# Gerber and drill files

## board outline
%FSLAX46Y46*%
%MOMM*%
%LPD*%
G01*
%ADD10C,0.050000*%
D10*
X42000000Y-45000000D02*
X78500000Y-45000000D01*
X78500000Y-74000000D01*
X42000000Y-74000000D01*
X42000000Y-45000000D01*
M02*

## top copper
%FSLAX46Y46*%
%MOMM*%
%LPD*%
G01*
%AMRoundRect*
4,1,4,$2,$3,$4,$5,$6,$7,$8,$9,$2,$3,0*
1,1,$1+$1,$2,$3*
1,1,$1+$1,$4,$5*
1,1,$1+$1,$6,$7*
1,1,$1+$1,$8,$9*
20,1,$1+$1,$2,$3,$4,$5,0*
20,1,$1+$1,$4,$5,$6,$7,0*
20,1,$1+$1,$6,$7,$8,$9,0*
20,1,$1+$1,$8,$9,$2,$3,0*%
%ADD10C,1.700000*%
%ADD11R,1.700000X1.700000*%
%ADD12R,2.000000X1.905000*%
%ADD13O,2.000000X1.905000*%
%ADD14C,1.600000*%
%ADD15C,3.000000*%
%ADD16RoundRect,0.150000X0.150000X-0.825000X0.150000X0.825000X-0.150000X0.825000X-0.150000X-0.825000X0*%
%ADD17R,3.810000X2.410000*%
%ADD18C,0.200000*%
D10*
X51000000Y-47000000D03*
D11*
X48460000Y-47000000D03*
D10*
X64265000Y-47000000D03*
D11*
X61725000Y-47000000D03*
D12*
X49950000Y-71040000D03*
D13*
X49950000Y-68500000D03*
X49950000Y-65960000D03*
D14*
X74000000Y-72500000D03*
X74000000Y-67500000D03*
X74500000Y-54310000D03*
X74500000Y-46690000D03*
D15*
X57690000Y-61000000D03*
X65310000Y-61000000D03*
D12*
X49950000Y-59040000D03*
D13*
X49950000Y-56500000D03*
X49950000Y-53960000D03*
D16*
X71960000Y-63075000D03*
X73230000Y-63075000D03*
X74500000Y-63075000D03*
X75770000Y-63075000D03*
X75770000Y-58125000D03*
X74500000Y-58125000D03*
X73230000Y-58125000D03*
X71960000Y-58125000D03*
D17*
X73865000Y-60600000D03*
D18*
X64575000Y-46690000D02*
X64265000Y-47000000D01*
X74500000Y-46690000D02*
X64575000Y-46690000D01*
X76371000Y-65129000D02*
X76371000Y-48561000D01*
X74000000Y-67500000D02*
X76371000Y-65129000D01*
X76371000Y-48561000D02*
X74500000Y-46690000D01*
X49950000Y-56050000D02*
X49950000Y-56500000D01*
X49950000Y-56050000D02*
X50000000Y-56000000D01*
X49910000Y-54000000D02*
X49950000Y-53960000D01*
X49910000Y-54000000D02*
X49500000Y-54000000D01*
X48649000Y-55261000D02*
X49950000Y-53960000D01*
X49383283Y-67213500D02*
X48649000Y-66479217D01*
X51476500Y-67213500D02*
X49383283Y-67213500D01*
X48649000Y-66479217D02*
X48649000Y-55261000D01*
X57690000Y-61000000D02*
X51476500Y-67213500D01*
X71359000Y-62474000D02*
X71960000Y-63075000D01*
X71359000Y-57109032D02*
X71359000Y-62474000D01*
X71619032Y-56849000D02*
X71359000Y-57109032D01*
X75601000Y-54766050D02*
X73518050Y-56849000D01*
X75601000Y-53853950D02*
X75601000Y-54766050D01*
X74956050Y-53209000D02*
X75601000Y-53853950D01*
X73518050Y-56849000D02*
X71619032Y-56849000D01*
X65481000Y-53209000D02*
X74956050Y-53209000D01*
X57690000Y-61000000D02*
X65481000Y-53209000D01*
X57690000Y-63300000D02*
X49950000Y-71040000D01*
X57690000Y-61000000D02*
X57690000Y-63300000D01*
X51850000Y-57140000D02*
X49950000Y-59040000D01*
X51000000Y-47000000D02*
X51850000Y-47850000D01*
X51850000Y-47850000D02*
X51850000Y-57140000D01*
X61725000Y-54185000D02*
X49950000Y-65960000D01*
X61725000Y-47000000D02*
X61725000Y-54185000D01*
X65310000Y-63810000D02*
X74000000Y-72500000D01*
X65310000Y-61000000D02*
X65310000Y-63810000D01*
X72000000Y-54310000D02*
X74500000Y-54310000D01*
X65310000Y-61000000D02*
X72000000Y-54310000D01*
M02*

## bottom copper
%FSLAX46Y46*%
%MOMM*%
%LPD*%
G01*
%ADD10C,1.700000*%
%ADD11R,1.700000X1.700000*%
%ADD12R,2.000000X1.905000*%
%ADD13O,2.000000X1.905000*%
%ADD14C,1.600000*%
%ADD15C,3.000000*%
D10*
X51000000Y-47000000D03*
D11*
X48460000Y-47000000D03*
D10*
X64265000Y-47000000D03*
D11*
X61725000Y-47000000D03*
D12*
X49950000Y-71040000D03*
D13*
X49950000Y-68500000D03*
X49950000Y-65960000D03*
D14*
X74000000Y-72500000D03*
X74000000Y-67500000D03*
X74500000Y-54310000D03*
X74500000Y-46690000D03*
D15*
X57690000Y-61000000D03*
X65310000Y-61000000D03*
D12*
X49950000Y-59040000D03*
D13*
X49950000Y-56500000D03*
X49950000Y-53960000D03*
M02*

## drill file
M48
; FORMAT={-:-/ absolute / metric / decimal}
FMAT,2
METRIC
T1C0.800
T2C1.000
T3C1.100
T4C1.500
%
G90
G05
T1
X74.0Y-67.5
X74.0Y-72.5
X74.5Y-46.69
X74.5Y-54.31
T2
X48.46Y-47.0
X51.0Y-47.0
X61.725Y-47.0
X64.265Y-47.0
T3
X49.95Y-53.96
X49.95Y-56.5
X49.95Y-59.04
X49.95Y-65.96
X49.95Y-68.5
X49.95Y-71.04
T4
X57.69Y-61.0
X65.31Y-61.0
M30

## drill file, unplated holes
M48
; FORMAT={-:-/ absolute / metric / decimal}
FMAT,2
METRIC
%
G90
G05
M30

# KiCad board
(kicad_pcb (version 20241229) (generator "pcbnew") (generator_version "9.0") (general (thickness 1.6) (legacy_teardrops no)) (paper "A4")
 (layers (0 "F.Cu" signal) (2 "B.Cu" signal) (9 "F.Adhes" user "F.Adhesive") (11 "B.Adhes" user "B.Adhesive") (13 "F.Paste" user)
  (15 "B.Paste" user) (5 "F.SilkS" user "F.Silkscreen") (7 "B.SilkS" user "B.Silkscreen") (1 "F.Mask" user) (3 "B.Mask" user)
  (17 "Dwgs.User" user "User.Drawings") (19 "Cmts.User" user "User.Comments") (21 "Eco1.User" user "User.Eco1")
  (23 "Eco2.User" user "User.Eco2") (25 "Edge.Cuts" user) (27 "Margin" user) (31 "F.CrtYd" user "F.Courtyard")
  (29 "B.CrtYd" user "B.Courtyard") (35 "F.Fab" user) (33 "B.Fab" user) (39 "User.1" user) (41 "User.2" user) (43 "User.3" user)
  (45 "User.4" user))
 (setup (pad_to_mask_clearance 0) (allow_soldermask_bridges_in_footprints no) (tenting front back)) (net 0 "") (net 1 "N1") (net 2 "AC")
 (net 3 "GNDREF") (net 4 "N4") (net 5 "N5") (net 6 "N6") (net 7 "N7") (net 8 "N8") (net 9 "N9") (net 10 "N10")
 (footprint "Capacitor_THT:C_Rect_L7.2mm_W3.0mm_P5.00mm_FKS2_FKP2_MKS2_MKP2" (layer "F.Cu") (at 74 72.5 90)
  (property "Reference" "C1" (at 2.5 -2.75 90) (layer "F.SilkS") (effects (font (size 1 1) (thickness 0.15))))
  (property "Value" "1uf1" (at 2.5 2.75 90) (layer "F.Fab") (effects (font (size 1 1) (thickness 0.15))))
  (pad "1" thru_hole circle (at 0 0 90) (size 1.6 1.6) (drill 0.8) (layers "*.Cu" "*.Mask") (remove_unused_layers no) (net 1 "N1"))
  (pad "2" thru_hole circle (at 5 0 90) (size 1.6 1.6) (drill 0.8) (layers "*.Cu" "*.Mask") (remove_unused_layers no) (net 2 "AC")))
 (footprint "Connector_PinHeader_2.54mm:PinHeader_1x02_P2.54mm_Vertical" (layer "F.Cu") (at 48.46 47 90)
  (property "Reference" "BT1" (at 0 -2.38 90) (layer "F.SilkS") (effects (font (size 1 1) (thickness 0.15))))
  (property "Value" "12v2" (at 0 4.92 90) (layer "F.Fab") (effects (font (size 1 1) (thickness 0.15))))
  (pad "1" thru_hole rect (at 0 0 90) (size 1.7 1.7) (drill 1) (layers "*.Cu" "*.Mask") (remove_unused_layers no) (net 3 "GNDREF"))
  (pad "2" thru_hole circle (at 0 2.54 90) (size 1.7 1.7) (drill 1) (layers "*.Cu" "*.Mask") (remove_unused_layers no) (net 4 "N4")))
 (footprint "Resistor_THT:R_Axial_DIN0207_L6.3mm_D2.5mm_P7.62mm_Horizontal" (layer "F.Cu") (at 74.5 54.31 90)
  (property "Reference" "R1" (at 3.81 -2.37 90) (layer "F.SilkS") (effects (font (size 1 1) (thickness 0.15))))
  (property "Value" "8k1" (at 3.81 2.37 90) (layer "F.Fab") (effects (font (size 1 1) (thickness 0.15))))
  (pad "1" thru_hole circle (at 0 0 90) (size 1.6 1.6) (drill 0.8) (layers "*.Cu" "*.Mask") (remove_unused_layers no) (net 1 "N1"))
  (pad "2" thru_hole circle (at 7.62 0 90) (size 1.6 1.6) (drill 0.8) (layers "*.Cu" "*.Mask") (remove_unused_layers no) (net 2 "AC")))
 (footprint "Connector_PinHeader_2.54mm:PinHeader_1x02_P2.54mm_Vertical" (layer "F.Cu") (at 61.725 47 90)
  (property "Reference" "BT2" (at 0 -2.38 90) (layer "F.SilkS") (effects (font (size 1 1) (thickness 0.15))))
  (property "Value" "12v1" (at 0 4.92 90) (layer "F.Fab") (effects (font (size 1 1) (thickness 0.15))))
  (pad "1" thru_hole rect (at 0 0 90) (size 1.7 1.7) (drill 1) (layers "*.Cu" "*.Mask") (remove_unused_layers no) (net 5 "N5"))
  (pad "2" thru_hole circle (at 0 2.54 90) (size 1.7 1.7) (drill 1) (layers "*.Cu" "*.Mask") (remove_unused_layers no) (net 2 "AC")))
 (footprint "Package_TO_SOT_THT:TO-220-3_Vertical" (layer "F.Cu") (at 49.95 71.04 90)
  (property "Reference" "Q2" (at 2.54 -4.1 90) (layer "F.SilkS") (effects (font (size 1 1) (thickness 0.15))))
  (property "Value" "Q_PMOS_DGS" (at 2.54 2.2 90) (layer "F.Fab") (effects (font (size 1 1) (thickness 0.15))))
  (pad "1" thru_hole rect (at 0 0 90) (size 1.905 2) (drill 1.1) (layers "*.Cu" "*.Mask") (remove_unused_layers no) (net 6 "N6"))
  (pad "2" thru_hole oval (at 2.54 0 90) (size 1.905 2) (drill 1.1) (layers "*.Cu" "*.Mask") (remove_unused_layers no) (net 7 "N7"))
  (pad "3" thru_hole oval (at 5.08 0 90) (size 1.905 2) (drill 1.1) (layers "*.Cu" "*.Mask") (remove_unused_layers no) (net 5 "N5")))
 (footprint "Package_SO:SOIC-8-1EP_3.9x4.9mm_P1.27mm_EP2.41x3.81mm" (layer "F.Cu") (at 73.865 60.6 90)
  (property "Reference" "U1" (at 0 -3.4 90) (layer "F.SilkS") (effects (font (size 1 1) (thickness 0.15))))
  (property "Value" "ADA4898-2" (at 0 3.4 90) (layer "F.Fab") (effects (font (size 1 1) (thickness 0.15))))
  (pad "" smd roundrect (at -0.6 -0.95 90) (size 0.97 1.54) (layers "F.Paste") (roundrect_rratio 0.25))
  (pad "" smd roundrect (at -0.6 0.95 90) (size 0.97 1.54) (layers "F.Paste") (roundrect_rratio 0.25))
  (pad "" smd roundrect (at 0.6 -0.95 90) (size 0.97 1.54) (layers "F.Paste") (roundrect_rratio 0.25))
  (pad "" smd roundrect (at 0.6 0.95 90) (size 0.97 1.54) (layers "F.Paste") (roundrect_rratio 0.25))
  (pad "1" smd roundrect (at -2.475 -1.905 90) (size 1.95 0.6) (layers "F.Cu" "F.Mask" "F.Paste") (roundrect_rratio 0.25) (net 6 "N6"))
  (pad "2" smd roundrect (at -2.475 -0.635 90) (size 1.95 0.6) (layers "F.Cu" "F.Mask" "F.Paste") (roundrect_rratio 0.25) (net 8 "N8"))
  (pad "3" smd roundrect (at -2.475 0.635 90) (size 1.95 0.6) (layers "F.Cu" "F.Mask" "F.Paste") (roundrect_rratio 0.25) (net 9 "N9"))
  (pad "4" smd roundrect (at -2.475 1.905 90) (size 1.95 0.6) (layers "F.Cu" "F.Mask" "F.Paste") (roundrect_rratio 0.25))
  (pad "5" smd roundrect (at 2.475 1.905 90) (size 1.95 0.6) (layers "F.Cu" "F.Mask" "F.Paste") (roundrect_rratio 0.25))
  (pad "6" smd roundrect (at 2.475 0.635 90) (size 1.95 0.6) (layers "F.Cu" "F.Mask" "F.Paste") (roundrect_rratio 0.25))
  (pad "7" smd roundrect (at 2.475 -0.635 90) (size 1.95 0.6) (layers "F.Cu" "F.Mask" "F.Paste") (roundrect_rratio 0.25))
  (pad "8" smd roundrect (at 2.475 -1.905 90) (size 1.95 0.6) (layers "F.Cu" "F.Mask" "F.Paste") (roundrect_rratio 0.25))
  (pad "9" smd rect (at 0 0 90) (size 2.41 3.81) (layers "F.Cu" "F.Mask") (zone_connect 2)))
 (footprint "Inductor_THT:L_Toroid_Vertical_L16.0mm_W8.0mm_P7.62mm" (layer "F.Cu") (at 57.69 61 90)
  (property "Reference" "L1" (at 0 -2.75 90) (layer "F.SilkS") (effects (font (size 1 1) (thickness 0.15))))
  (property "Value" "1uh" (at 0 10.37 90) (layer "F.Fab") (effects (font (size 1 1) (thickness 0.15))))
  (pad "1" thru_hole circle (at 0 0 90) (size 3 3) (drill 1.5) (layers "*.Cu" "*.Mask") (remove_unused_layers no) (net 6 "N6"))
  (pad "2" thru_hole circle (at 0 7.62 90) (size 3 3) (drill 1.5) (layers "*.Cu" "*.Mask") (remove_unused_layers no) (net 1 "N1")))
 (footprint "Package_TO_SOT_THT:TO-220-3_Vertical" (layer "F.Cu") (at 49.95 59.04 90)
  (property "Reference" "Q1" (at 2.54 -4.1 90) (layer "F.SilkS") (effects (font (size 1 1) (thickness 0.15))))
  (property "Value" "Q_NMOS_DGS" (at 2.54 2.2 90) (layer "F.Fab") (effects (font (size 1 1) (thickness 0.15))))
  (pad "1" thru_hole rect (at 0 0 90) (size 1.905 2) (drill 1.1) (layers "*.Cu" "*.Mask") (remove_unused_layers no) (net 4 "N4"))
  (pad "2" thru_hole oval (at 2.54 0 90) (size 1.905 2) (drill 1.1) (layers "*.Cu" "*.Mask") (remove_unused_layers no) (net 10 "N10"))
  (pad "3" thru_hole oval (at 5.08 0 90) (size 1.905 2) (drill 1.1) (layers "*.Cu" "*.Mask") (remove_unused_layers no) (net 6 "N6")))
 (gr_rect (start 42 45) (end 78.5 74) (stroke (width 0.05) (type default)) (fill no) (layer "Edge.Cuts"))
 (segment (start 73 60.5) (end 73.541968 60.5) (width 0.2) (layer "F.Cu") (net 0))
 (segment (start 75.77 58.125) (end 71.96 58.125) (width 0.2) (layer "F.Cu") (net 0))
 (segment (start 73.1 60.6) (end 73 60.5) (width 0.2) (layer "F.Cu") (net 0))
 (segment (start 75.77 62.728032) (end 75.77 63.075) (width 0.2) (layer "F.Cu") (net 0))
 (segment (start 73.865 60.6) (end 73.1 60.6) (width 0.2) (layer "F.Cu") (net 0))
 (segment (start 73.541968 60.5) (end 75.77 62.728032) (width 0.2) (layer "F.Cu") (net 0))
 (segment (start 61.725 47) (end 61.725 54.185) (width 0.2) (layer "F.Cu") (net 5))
 (segment (start 61.725 54.185) (end 49.95 65.96) (width 0.2) (layer "F.Cu") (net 5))
 (segment (start 76.371 48.561) (end 74.5 46.69) (width 0.2) (layer "F.Cu") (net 2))
 (segment (start 74.5 46.69) (end 64.575 46.69) (width 0.2) (layer "F.Cu") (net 2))
 (segment (start 76.371 65.129) (end 76.371 48.561) (width 0.2) (layer "F.Cu") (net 2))
 (segment (start 64.575 46.69) (end 64.265 47) (width 0.2) (layer "F.Cu") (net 2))
 (segment (start 74 67.5) (end 76.371 65.129) (width 0.2) (layer "F.Cu") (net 2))
 (segment (start 65.31 63.81) (end 74 72.5) (width 0.2) (layer "F.Cu") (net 1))
 (segment (start 72 54.31) (end 74.5 54.31) (width 0.2) (layer "F.Cu") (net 1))
 (segment (start 65.31 61) (end 72 54.31) (width 0.2) (layer "F.Cu") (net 1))
 (segment (start 65.31 61) (end 65.31 63.81) (width 0.2) (layer "F.Cu") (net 1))
 (segment (start 57.69 61) (end 65.481 53.209) (width 0.2) (layer "F.Cu") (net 6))
 (segment (start 48.649 66.479217) (end 48.649 55.261) (width 0.2) (layer "F.Cu") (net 6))
 (segment (start 57.69 61) (end 57.69 63.3) (width 0.2) (layer "F.Cu") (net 6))
 (segment (start 51.4765 67.2135) (end 49.383283 67.2135) (width 0.2) (layer "F.Cu") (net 6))
 (segment (start 75.601 53.85395) (end 75.601 54.76605) (width 0.2) (layer "F.Cu") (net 6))
 (segment (start 71.359 57.109032) (end 71.359 62.474) (width 0.2) (layer "F.Cu") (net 6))
 (segment (start 57.69 63.3) (end 49.95 71.04) (width 0.2) (layer "F.Cu") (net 6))
 (segment (start 71.619032 56.849) (end 71.359 57.109032) (width 0.2) (layer "F.Cu") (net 6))
 (segment (start 49.91 54) (end 49.95 53.96) (width 0.2) (layer "F.Cu") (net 6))
 (segment (start 49.383283 67.2135) (end 48.649 66.479217) (width 0.2) (layer "F.Cu") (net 6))
 (segment (start 49.91 54) (end 49.5 54) (width 0.2) (layer "F.Cu") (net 6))
 (segment (start 74.95605 53.209) (end 75.601 53.85395) (width 0.2) (layer "F.Cu") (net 6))
 (segment (start 65.481 53.209) (end 74.95605 53.209) (width 0.2) (layer "F.Cu") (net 6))
 (segment (start 71.359 62.474) (end 71.96 63.075) (width 0.2) (layer "F.Cu") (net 6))
 (segment (start 75.601 54.76605) (end 73.51805 56.849) (width 0.2) (layer "F.Cu") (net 6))
 (segment (start 48.649 55.261) (end 49.95 53.96) (width 0.2) (layer "F.Cu") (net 6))
 (segment (start 73.51805 56.849) (end 71.619032 56.849) (width 0.2) (layer "F.Cu") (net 6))
 (segment (start 57.69 61) (end 51.4765 67.2135) (width 0.2) (layer "F.Cu") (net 6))
 (segment (start 51.85 57.14) (end 49.95 59.04) (width 0.2) (layer "F.Cu") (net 4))
 (segment (start 51.85 47.85) (end 51.85 57.14) (width 0.2) (layer "F.Cu") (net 4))
 (segment (start 51 47) (end 51.85 47.85) (width 0.2) (layer "F.Cu") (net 4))
 (segment (start 49.95 56.05) (end 49.95 56.5) (width 0.2) (layer "F.Cu") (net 10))
 (segment (start 49.95 56.05) (end 50 56) (width 0.2) (layer "F.Cu") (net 10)))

